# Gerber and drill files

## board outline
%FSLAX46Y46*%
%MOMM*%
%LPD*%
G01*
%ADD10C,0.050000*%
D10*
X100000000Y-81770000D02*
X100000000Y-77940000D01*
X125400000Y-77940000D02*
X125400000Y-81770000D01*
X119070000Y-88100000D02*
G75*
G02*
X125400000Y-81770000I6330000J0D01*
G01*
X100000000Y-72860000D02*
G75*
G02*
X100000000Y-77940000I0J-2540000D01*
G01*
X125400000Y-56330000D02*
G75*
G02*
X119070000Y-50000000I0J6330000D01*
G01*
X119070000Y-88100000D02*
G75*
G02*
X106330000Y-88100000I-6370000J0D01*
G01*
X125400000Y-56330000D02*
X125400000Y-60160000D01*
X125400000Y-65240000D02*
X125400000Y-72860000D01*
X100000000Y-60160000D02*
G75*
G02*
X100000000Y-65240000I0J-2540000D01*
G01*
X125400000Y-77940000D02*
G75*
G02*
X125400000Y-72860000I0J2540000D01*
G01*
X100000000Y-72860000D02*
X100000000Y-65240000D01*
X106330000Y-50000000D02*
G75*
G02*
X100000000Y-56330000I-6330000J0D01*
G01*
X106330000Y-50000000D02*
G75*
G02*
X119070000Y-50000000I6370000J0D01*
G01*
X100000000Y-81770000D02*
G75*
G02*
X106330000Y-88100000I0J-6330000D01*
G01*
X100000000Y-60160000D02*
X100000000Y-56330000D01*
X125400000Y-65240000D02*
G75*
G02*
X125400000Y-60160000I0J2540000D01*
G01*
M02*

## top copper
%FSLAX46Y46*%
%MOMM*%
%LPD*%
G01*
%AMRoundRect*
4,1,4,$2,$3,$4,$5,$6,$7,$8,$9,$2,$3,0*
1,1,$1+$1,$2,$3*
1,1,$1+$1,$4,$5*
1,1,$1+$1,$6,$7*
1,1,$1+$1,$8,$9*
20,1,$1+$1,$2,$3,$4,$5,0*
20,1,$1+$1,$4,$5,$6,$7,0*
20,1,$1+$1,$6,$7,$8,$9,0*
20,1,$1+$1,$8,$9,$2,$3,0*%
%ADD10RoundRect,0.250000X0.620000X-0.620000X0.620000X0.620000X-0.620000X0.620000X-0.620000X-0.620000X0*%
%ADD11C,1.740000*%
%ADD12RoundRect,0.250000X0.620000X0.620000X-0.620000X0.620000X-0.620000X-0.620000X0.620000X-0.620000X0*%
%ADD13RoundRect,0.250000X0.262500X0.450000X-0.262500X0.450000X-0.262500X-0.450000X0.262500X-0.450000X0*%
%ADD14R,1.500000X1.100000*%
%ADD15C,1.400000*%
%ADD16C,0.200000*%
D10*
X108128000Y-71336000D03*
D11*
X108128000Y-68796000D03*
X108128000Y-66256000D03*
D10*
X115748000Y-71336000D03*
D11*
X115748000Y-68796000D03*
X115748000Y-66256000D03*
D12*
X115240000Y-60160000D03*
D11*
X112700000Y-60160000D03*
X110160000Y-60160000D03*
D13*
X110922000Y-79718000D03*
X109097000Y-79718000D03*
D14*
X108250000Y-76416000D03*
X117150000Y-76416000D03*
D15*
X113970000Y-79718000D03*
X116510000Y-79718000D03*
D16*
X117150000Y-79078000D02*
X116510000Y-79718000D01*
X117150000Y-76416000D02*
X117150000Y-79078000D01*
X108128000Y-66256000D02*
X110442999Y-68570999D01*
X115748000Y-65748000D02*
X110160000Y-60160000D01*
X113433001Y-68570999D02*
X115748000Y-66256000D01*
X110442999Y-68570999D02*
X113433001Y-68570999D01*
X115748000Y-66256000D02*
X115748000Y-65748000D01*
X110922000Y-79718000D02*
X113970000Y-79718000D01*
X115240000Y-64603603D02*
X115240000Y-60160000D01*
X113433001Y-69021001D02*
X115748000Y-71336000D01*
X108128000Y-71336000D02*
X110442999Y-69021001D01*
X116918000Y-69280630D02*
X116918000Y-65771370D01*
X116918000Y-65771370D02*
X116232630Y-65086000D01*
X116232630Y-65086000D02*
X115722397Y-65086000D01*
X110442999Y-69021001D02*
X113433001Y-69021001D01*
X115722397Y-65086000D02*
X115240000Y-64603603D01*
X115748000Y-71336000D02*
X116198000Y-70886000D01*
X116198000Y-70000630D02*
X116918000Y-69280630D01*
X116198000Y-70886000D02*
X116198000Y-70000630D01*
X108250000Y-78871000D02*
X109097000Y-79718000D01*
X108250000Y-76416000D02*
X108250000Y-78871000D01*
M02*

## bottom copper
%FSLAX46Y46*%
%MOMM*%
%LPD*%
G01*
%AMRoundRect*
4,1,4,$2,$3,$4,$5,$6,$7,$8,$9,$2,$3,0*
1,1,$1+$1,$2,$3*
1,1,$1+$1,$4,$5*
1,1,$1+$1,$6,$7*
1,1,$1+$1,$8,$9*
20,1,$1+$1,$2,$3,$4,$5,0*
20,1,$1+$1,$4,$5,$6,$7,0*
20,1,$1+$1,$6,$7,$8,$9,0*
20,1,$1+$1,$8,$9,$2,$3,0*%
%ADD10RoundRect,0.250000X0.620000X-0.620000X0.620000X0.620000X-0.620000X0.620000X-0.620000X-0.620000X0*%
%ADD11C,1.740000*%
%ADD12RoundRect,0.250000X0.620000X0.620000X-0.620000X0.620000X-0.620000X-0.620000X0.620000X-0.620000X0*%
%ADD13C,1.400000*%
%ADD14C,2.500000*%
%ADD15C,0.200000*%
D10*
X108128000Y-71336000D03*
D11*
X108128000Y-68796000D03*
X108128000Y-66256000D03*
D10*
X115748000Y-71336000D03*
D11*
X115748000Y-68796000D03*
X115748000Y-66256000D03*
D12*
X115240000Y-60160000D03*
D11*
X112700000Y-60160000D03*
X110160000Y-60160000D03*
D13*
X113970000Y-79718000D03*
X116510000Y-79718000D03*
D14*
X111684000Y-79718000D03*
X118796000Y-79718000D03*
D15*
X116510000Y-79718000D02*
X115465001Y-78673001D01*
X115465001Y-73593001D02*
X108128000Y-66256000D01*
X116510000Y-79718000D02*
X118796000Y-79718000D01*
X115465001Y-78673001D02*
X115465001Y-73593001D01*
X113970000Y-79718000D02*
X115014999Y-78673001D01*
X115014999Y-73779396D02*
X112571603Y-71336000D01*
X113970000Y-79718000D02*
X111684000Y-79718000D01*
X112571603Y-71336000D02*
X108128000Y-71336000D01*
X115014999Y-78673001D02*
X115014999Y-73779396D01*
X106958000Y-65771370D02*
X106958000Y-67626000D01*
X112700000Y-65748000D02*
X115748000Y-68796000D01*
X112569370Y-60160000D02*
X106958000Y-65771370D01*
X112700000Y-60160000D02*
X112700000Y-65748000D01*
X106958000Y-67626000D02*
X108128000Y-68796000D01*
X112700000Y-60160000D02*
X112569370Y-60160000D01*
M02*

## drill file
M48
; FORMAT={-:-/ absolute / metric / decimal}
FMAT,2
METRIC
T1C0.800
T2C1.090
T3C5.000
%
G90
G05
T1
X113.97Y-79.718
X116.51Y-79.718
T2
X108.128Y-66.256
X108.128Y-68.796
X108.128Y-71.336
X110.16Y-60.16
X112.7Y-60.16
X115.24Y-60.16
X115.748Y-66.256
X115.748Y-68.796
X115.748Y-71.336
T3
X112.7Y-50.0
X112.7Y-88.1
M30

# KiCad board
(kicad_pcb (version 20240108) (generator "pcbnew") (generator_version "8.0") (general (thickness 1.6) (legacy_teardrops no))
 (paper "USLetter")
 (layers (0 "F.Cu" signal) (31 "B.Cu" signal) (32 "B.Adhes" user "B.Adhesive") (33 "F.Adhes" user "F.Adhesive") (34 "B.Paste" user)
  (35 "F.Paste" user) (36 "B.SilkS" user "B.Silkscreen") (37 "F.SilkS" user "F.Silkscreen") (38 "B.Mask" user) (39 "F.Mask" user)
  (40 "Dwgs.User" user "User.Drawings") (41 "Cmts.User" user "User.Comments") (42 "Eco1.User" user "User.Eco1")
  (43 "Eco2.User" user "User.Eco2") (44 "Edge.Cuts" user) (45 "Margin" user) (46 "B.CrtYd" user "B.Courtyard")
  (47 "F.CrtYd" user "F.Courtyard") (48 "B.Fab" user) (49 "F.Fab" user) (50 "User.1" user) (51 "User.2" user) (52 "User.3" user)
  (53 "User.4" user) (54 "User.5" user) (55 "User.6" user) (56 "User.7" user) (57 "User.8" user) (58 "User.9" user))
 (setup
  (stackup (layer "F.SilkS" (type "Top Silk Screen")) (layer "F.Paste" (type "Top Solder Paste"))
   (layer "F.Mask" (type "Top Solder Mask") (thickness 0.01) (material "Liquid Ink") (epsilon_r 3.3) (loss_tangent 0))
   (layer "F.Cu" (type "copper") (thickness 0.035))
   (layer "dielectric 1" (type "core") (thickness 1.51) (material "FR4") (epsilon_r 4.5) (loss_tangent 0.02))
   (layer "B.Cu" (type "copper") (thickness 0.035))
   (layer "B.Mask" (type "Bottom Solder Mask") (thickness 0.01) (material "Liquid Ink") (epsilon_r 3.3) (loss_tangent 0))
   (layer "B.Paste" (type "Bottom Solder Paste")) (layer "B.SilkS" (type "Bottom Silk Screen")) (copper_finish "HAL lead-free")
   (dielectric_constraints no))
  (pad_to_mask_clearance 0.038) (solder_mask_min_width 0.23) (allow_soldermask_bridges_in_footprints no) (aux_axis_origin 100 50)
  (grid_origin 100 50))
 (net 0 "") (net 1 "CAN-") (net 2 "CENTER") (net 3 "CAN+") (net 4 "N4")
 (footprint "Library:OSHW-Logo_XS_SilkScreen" (layer "F.Cu") (at 103.81 79.718)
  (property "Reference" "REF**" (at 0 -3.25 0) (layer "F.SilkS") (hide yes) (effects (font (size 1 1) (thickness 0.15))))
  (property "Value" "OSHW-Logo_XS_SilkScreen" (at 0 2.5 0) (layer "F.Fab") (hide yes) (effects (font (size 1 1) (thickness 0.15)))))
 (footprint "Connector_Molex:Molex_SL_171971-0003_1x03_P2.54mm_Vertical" (layer "F.Cu") (at 108.128 71.336 90)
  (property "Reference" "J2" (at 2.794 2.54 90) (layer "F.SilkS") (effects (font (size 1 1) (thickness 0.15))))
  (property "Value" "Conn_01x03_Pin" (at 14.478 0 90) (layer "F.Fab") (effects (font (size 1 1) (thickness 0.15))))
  (pad "1" thru_hole roundrect (at 0 0 90) (size 1.74 1.74) (drill 1.09) (layers "*.Cu" "*.Mask") (remove_unused_layers no)
   (roundrect_rratio 0.143678) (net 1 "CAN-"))
  (pad "2" thru_hole circle (at 2.54 0 90) (size 1.74 1.74) (drill 1.09) (layers "*.Cu" "*.Mask") (remove_unused_layers no) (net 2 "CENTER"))
  (pad "3" thru_hole circle (at 5.08 0 90) (size 1.74 1.74) (drill 1.09) (layers "*.Cu" "*.Mask") (remove_unused_layers no) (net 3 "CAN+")))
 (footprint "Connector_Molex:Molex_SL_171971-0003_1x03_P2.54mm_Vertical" (layer "F.Cu") (at 115.748 71.336 90)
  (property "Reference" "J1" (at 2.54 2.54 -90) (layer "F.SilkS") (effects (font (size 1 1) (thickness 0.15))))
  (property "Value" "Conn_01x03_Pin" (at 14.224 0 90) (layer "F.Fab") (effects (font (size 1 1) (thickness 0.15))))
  (pad "1" thru_hole roundrect (at 0 0 90) (size 1.74 1.74) (drill 1.09) (layers "*.Cu" "*.Mask") (remove_unused_layers no)
   (roundrect_rratio 0.143678) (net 1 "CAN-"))
  (pad "2" thru_hole circle (at 2.54 0 90) (size 1.74 1.74) (drill 1.09) (layers "*.Cu" "*.Mask") (remove_unused_layers no) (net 2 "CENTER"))
  (pad "3" thru_hole circle (at 5.08 0 90) (size 1.74 1.74) (drill 1.09) (layers "*.Cu" "*.Mask") (remove_unused_layers no) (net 3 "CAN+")))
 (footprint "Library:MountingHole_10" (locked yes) (layer "F.Cu") (at 112.7 88.1)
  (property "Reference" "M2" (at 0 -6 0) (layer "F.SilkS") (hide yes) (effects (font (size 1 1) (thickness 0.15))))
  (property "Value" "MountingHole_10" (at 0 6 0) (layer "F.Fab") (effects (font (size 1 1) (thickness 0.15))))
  (pad "" np_thru_hole circle (at 0 0) (size 5 5) (drill 5) (layers "*.Cu" "*.Mask")))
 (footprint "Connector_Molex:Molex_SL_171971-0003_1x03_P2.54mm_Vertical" (layer "F.Cu") (at 115.24 60.16 180)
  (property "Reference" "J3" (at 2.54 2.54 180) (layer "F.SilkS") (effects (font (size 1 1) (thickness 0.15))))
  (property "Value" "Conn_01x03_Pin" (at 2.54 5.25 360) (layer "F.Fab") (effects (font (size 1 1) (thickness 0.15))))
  (pad "1" thru_hole roundrect (at 0 0 180) (size 1.74 1.74) (drill 1.09) (layers "*.Cu" "*.Mask") (remove_unused_layers no)
   (roundrect_rratio 0.143678) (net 1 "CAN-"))
  (pad "2" thru_hole circle (at 2.54 0 180) (size 1.74 1.74) (drill 1.09) (layers "*.Cu" "*.Mask") (remove_unused_layers no)
   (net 2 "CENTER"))
  (pad "3" thru_hole circle (at 5.08 0 180) (size 1.74 1.74) (drill 1.09) (layers "*.Cu" "*.Mask") (remove_unused_layers no) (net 3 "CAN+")))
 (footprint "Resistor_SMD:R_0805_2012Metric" (layer "F.Cu") (at 110.0095 79.718 180)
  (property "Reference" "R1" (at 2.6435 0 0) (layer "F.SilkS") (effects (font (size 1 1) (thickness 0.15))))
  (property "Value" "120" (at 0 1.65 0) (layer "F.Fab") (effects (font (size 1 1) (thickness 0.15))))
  (pad "1" smd roundrect (at -0.9125 0 180) (size 1.025 1.4) (layers "F.Cu" "F.Paste" "F.Mask") (roundrect_rratio 0.243902) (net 1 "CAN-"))
  (pad "2" smd roundrect (at 0.9125 0 180) (size 1.025 1.4) (layers "F.Cu" "F.Paste" "F.Mask") (roundrect_rratio 0.243902) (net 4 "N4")))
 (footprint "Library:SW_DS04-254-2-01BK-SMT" (layer "F.Cu") (at 112.7 76.416)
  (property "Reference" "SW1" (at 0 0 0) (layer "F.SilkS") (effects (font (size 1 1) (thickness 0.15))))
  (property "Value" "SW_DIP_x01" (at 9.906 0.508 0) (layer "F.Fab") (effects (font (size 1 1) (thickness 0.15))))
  (pad "1" smd rect (at -4.45 0) (size 1.5 1.1) (layers "F.Cu" "F.Paste" "F.Mask") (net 4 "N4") (solder_mask_margin 0.102))
  (pad "2" smd rect (at 4.45 0) (size 1.5 1.1) (layers "F.Cu" "F.Paste" "F.Mask") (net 3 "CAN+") (solder_mask_margin 0.102)))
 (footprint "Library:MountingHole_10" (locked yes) (layer "F.Cu") (at 112.7 50)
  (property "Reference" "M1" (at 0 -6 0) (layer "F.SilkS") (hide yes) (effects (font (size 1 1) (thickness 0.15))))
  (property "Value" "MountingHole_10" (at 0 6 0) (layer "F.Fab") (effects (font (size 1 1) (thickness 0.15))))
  (pad "" np_thru_hole circle (at 0 0) (size 5 5) (drill 5) (layers "*.Cu" "*.Mask")))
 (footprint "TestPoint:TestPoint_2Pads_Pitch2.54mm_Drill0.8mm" (layer "F.Cu") (at 113.97 79.718)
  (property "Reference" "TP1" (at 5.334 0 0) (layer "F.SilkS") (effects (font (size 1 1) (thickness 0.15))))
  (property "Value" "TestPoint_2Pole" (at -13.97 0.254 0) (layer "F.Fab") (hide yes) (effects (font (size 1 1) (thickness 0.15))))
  (pad "1" thru_hole circle (at 0 0) (size 1.4 1.4) (drill 0.8) (layers "*.Cu" "*.Mask") (remove_unused_layers no) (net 1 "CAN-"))
  (pad "2" thru_hole circle (at 2.54 0) (size 1.4 1.4) (drill 0.8) (layers "*.Cu" "*.Mask") (remove_unused_layers no) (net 3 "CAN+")))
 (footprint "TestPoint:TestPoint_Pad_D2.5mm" (layer "B.Cu") (at 111.684 79.718 180)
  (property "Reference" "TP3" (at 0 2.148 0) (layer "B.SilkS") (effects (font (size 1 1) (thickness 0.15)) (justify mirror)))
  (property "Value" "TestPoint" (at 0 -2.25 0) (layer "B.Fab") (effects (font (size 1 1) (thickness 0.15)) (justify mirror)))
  (pad "1" smd circle (at 0 0 180) (size 2.5 2.5) (layers "B.Cu" "B.Mask") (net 1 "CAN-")))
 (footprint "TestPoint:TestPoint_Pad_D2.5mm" (layer "B.Cu") (at 118.796 79.718 180)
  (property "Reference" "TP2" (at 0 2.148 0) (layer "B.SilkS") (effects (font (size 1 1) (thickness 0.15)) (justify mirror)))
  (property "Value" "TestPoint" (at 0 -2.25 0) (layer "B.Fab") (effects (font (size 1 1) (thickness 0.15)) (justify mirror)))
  (pad "1" smd circle (at 0 0 180) (size 2.5 2.5) (layers "B.Cu" "B.Mask") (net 3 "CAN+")))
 (gr_line (start 100 81.77) (end 100 77.94) (locked yes) (stroke (width 0.05) (type default)) (layer "Edge.Cuts"))
 (gr_line (start 125.4 77.94) (end 125.4 81.77) (locked yes) (stroke (width 0.05) (type default)) (layer "Edge.Cuts"))
 (gr_arc (start 119.07 88.1) (mid 120.924014 83.624014) (end 125.4 81.77) (locked yes) (stroke (width 0.05) (type default))
  (layer "Edge.Cuts"))
 (gr_arc (start 100 72.86) (mid 102.54 75.4) (end 100 77.94) (locked yes) (stroke (width 0.05) (type default)) (layer "Edge.Cuts"))
 (gr_arc (start 125.4 56.33) (mid 120.924014 54.475986) (end 119.07 50) (locked yes) (stroke (width 0.05) (type default))
  (layer "Edge.Cuts"))
 (gr_arc (start 119.07 88.1) (mid 112.7 94.47) (end 106.33 88.1) (locked yes) (stroke (width 0.05) (type default)) (layer "Edge.Cuts"))
 (gr_line (start 125.4 56.33) (end 125.4 60.16) (locked yes) (stroke (width 0.05) (type default)) (layer "Edge.Cuts"))
 (gr_line (start 125.4 65.24) (end 125.4 72.86) (locked yes) (stroke (width 0.05) (type default)) (layer "Edge.Cuts"))
 (gr_arc (start 100 60.16) (mid 102.54 62.7) (end 100 65.24) (locked yes) (stroke (width 0.05) (type default)) (layer "Edge.Cuts"))
 (gr_arc (start 125.4 77.94) (mid 122.86 75.4) (end 125.4 72.86) (locked yes) (stroke (width 0.05) (type default)) (layer "Edge.Cuts"))
 (gr_line (start 100 72.86) (end 100 65.24) (locked yes) (stroke (width 0.05) (type default)) (layer "Edge.Cuts"))
 (gr_arc (start 106.33 50) (mid 104.475986 54.475986) (end 100 56.33) (locked yes) (stroke (width 0.05) (type default)) (layer "Edge.Cuts"))
 (gr_arc (start 106.33 50) (mid 112.7 43.63) (end 119.07 50) (locked yes) (stroke (width 0.05) (type default)) (layer "Edge.Cuts"))
 (gr_arc (start 100 81.77) (mid 104.475986 83.624014) (end 106.33 88.1) (locked yes) (stroke (width 0.05) (type default))
  (layer "Edge.Cuts"))
 (gr_line (start 100 60.16) (end 100 56.33) (locked yes) (stroke (width 0.05) (type default)) (layer "Edge.Cuts"))
 (gr_arc (start 125.4 65.24) (mid 122.86 62.7) (end 125.4 60.16) (locked yes) (stroke (width 0.05) (type default)) (layer "Edge.Cuts"))
 (segment (start 117.15 79.078) (end 116.51 79.718) (width 0.2) (layer "F.Cu") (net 3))
 (segment (start 117.15 76.416) (end 117.15 79.078) (width 0.2) (layer "F.Cu") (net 3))
 (segment (start 108.128 66.256) (end 110.442999 68.570999) (width 0.2) (layer "F.Cu") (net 3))
 (segment (start 115.748 65.748) (end 110.16 60.16) (width 0.2) (layer "F.Cu") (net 3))
 (segment (start 113.433001 68.570999) (end 115.748 66.256) (width 0.2) (layer "F.Cu") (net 3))
 (segment (start 110.442999 68.570999) (end 113.433001 68.570999) (width 0.2) (layer "F.Cu") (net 3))
 (segment (start 115.748 66.256) (end 115.748 65.748) (width 0.2) (layer "F.Cu") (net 3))
 (segment (start 116.51 79.718) (end 115.465001 78.673001) (width 0.2) (layer "B.Cu") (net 3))
 (segment (start 115.465001 73.593001) (end 108.128 66.256) (width 0.2) (layer "B.Cu") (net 3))
 (segment (start 116.51 79.718) (end 118.796 79.718) (width 0.2) (layer "B.Cu") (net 3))
 (segment (start 115.465001 78.673001) (end 115.465001 73.593001) (width 0.2) (layer "B.Cu") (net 3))
 (segment (start 110.922 79.718) (end 113.97 79.718) (width 0.2) (layer "F.Cu") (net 1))
 (segment (start 115.24 64.603603) (end 115.24 60.16) (width 0.2) (layer "F.Cu") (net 1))
 (segment (start 113.433001 69.021001) (end 115.748 71.336) (width 0.2) (layer "F.Cu") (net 1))
 (segment (start 108.128 71.336) (end 110.442999 69.021001) (width 0.2) (layer "F.Cu") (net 1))
 (segment (start 116.918 69.28063) (end 116.918 65.77137) (width 0.2) (layer "F.Cu") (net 1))
 (segment (start 116.918 65.77137) (end 116.23263 65.086) (width 0.2) (layer "F.Cu") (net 1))
 (segment (start 116.23263 65.086) (end 115.722397 65.086) (width 0.2) (layer "F.Cu") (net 1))
 (segment (start 110.442999 69.021001) (end 113.433001 69.021001) (width 0.2) (layer "F.Cu") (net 1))
 (segment (start 115.722397 65.086) (end 115.24 64.603603) (width 0.2) (layer "F.Cu") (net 1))
 (segment (start 115.748 71.336) (end 116.198 70.886) (width 0.2) (layer "F.Cu") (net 1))
 (segment (start 116.198 70.00063) (end 116.918 69.28063) (width 0.2) (layer "F.Cu") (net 1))
 (segment (start 116.198 70.886) (end 116.198 70.00063) (width 0.2) (layer "F.Cu") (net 1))
 (segment (start 113.97 79.718) (end 115.014999 78.673001) (width 0.2) (layer "B.Cu") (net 1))
 (segment (start 115.014999 73.779396) (end 112.571603 71.336) (width 0.2) (layer "B.Cu") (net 1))
 (segment (start 113.97 79.718) (end 111.684 79.718) (width 0.2) (layer "B.Cu") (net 1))
 (segment (start 112.571603 71.336) (end 108.128 71.336) (width 0.2) (layer "B.Cu") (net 1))
 (segment (start 115.014999 78.673001) (end 115.014999 73.779396) (width 0.2) (layer "B.Cu") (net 1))
 (segment (start 106.958 65.77137) (end 106.958 67.626) (width 0.2) (layer "B.Cu") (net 2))
 (segment (start 112.7 65.748) (end 115.748 68.796) (width 0.2) (layer "B.Cu") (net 2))
 (segment (start 112.56937 60.16) (end 106.958 65.77137) (width 0.2) (layer "B.Cu") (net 2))
 (segment (start 112.7 60.16) (end 112.7 65.748) (width 0.2) (layer "B.Cu") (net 2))
 (segment (start 106.958 67.626) (end 108.128 68.796) (width 0.2) (layer "B.Cu") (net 2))
 (segment (start 112.7 60.16) (end 112.56937 60.16) (width 0.2) (layer "B.Cu") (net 2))
 (segment (start 108.25 78.871) (end 109.097 79.718) (width 0.2) (layer "F.Cu") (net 4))
 (segment (start 108.25 76.416) (end 108.25 78.871) (width 0.2) (layer "F.Cu") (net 4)))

